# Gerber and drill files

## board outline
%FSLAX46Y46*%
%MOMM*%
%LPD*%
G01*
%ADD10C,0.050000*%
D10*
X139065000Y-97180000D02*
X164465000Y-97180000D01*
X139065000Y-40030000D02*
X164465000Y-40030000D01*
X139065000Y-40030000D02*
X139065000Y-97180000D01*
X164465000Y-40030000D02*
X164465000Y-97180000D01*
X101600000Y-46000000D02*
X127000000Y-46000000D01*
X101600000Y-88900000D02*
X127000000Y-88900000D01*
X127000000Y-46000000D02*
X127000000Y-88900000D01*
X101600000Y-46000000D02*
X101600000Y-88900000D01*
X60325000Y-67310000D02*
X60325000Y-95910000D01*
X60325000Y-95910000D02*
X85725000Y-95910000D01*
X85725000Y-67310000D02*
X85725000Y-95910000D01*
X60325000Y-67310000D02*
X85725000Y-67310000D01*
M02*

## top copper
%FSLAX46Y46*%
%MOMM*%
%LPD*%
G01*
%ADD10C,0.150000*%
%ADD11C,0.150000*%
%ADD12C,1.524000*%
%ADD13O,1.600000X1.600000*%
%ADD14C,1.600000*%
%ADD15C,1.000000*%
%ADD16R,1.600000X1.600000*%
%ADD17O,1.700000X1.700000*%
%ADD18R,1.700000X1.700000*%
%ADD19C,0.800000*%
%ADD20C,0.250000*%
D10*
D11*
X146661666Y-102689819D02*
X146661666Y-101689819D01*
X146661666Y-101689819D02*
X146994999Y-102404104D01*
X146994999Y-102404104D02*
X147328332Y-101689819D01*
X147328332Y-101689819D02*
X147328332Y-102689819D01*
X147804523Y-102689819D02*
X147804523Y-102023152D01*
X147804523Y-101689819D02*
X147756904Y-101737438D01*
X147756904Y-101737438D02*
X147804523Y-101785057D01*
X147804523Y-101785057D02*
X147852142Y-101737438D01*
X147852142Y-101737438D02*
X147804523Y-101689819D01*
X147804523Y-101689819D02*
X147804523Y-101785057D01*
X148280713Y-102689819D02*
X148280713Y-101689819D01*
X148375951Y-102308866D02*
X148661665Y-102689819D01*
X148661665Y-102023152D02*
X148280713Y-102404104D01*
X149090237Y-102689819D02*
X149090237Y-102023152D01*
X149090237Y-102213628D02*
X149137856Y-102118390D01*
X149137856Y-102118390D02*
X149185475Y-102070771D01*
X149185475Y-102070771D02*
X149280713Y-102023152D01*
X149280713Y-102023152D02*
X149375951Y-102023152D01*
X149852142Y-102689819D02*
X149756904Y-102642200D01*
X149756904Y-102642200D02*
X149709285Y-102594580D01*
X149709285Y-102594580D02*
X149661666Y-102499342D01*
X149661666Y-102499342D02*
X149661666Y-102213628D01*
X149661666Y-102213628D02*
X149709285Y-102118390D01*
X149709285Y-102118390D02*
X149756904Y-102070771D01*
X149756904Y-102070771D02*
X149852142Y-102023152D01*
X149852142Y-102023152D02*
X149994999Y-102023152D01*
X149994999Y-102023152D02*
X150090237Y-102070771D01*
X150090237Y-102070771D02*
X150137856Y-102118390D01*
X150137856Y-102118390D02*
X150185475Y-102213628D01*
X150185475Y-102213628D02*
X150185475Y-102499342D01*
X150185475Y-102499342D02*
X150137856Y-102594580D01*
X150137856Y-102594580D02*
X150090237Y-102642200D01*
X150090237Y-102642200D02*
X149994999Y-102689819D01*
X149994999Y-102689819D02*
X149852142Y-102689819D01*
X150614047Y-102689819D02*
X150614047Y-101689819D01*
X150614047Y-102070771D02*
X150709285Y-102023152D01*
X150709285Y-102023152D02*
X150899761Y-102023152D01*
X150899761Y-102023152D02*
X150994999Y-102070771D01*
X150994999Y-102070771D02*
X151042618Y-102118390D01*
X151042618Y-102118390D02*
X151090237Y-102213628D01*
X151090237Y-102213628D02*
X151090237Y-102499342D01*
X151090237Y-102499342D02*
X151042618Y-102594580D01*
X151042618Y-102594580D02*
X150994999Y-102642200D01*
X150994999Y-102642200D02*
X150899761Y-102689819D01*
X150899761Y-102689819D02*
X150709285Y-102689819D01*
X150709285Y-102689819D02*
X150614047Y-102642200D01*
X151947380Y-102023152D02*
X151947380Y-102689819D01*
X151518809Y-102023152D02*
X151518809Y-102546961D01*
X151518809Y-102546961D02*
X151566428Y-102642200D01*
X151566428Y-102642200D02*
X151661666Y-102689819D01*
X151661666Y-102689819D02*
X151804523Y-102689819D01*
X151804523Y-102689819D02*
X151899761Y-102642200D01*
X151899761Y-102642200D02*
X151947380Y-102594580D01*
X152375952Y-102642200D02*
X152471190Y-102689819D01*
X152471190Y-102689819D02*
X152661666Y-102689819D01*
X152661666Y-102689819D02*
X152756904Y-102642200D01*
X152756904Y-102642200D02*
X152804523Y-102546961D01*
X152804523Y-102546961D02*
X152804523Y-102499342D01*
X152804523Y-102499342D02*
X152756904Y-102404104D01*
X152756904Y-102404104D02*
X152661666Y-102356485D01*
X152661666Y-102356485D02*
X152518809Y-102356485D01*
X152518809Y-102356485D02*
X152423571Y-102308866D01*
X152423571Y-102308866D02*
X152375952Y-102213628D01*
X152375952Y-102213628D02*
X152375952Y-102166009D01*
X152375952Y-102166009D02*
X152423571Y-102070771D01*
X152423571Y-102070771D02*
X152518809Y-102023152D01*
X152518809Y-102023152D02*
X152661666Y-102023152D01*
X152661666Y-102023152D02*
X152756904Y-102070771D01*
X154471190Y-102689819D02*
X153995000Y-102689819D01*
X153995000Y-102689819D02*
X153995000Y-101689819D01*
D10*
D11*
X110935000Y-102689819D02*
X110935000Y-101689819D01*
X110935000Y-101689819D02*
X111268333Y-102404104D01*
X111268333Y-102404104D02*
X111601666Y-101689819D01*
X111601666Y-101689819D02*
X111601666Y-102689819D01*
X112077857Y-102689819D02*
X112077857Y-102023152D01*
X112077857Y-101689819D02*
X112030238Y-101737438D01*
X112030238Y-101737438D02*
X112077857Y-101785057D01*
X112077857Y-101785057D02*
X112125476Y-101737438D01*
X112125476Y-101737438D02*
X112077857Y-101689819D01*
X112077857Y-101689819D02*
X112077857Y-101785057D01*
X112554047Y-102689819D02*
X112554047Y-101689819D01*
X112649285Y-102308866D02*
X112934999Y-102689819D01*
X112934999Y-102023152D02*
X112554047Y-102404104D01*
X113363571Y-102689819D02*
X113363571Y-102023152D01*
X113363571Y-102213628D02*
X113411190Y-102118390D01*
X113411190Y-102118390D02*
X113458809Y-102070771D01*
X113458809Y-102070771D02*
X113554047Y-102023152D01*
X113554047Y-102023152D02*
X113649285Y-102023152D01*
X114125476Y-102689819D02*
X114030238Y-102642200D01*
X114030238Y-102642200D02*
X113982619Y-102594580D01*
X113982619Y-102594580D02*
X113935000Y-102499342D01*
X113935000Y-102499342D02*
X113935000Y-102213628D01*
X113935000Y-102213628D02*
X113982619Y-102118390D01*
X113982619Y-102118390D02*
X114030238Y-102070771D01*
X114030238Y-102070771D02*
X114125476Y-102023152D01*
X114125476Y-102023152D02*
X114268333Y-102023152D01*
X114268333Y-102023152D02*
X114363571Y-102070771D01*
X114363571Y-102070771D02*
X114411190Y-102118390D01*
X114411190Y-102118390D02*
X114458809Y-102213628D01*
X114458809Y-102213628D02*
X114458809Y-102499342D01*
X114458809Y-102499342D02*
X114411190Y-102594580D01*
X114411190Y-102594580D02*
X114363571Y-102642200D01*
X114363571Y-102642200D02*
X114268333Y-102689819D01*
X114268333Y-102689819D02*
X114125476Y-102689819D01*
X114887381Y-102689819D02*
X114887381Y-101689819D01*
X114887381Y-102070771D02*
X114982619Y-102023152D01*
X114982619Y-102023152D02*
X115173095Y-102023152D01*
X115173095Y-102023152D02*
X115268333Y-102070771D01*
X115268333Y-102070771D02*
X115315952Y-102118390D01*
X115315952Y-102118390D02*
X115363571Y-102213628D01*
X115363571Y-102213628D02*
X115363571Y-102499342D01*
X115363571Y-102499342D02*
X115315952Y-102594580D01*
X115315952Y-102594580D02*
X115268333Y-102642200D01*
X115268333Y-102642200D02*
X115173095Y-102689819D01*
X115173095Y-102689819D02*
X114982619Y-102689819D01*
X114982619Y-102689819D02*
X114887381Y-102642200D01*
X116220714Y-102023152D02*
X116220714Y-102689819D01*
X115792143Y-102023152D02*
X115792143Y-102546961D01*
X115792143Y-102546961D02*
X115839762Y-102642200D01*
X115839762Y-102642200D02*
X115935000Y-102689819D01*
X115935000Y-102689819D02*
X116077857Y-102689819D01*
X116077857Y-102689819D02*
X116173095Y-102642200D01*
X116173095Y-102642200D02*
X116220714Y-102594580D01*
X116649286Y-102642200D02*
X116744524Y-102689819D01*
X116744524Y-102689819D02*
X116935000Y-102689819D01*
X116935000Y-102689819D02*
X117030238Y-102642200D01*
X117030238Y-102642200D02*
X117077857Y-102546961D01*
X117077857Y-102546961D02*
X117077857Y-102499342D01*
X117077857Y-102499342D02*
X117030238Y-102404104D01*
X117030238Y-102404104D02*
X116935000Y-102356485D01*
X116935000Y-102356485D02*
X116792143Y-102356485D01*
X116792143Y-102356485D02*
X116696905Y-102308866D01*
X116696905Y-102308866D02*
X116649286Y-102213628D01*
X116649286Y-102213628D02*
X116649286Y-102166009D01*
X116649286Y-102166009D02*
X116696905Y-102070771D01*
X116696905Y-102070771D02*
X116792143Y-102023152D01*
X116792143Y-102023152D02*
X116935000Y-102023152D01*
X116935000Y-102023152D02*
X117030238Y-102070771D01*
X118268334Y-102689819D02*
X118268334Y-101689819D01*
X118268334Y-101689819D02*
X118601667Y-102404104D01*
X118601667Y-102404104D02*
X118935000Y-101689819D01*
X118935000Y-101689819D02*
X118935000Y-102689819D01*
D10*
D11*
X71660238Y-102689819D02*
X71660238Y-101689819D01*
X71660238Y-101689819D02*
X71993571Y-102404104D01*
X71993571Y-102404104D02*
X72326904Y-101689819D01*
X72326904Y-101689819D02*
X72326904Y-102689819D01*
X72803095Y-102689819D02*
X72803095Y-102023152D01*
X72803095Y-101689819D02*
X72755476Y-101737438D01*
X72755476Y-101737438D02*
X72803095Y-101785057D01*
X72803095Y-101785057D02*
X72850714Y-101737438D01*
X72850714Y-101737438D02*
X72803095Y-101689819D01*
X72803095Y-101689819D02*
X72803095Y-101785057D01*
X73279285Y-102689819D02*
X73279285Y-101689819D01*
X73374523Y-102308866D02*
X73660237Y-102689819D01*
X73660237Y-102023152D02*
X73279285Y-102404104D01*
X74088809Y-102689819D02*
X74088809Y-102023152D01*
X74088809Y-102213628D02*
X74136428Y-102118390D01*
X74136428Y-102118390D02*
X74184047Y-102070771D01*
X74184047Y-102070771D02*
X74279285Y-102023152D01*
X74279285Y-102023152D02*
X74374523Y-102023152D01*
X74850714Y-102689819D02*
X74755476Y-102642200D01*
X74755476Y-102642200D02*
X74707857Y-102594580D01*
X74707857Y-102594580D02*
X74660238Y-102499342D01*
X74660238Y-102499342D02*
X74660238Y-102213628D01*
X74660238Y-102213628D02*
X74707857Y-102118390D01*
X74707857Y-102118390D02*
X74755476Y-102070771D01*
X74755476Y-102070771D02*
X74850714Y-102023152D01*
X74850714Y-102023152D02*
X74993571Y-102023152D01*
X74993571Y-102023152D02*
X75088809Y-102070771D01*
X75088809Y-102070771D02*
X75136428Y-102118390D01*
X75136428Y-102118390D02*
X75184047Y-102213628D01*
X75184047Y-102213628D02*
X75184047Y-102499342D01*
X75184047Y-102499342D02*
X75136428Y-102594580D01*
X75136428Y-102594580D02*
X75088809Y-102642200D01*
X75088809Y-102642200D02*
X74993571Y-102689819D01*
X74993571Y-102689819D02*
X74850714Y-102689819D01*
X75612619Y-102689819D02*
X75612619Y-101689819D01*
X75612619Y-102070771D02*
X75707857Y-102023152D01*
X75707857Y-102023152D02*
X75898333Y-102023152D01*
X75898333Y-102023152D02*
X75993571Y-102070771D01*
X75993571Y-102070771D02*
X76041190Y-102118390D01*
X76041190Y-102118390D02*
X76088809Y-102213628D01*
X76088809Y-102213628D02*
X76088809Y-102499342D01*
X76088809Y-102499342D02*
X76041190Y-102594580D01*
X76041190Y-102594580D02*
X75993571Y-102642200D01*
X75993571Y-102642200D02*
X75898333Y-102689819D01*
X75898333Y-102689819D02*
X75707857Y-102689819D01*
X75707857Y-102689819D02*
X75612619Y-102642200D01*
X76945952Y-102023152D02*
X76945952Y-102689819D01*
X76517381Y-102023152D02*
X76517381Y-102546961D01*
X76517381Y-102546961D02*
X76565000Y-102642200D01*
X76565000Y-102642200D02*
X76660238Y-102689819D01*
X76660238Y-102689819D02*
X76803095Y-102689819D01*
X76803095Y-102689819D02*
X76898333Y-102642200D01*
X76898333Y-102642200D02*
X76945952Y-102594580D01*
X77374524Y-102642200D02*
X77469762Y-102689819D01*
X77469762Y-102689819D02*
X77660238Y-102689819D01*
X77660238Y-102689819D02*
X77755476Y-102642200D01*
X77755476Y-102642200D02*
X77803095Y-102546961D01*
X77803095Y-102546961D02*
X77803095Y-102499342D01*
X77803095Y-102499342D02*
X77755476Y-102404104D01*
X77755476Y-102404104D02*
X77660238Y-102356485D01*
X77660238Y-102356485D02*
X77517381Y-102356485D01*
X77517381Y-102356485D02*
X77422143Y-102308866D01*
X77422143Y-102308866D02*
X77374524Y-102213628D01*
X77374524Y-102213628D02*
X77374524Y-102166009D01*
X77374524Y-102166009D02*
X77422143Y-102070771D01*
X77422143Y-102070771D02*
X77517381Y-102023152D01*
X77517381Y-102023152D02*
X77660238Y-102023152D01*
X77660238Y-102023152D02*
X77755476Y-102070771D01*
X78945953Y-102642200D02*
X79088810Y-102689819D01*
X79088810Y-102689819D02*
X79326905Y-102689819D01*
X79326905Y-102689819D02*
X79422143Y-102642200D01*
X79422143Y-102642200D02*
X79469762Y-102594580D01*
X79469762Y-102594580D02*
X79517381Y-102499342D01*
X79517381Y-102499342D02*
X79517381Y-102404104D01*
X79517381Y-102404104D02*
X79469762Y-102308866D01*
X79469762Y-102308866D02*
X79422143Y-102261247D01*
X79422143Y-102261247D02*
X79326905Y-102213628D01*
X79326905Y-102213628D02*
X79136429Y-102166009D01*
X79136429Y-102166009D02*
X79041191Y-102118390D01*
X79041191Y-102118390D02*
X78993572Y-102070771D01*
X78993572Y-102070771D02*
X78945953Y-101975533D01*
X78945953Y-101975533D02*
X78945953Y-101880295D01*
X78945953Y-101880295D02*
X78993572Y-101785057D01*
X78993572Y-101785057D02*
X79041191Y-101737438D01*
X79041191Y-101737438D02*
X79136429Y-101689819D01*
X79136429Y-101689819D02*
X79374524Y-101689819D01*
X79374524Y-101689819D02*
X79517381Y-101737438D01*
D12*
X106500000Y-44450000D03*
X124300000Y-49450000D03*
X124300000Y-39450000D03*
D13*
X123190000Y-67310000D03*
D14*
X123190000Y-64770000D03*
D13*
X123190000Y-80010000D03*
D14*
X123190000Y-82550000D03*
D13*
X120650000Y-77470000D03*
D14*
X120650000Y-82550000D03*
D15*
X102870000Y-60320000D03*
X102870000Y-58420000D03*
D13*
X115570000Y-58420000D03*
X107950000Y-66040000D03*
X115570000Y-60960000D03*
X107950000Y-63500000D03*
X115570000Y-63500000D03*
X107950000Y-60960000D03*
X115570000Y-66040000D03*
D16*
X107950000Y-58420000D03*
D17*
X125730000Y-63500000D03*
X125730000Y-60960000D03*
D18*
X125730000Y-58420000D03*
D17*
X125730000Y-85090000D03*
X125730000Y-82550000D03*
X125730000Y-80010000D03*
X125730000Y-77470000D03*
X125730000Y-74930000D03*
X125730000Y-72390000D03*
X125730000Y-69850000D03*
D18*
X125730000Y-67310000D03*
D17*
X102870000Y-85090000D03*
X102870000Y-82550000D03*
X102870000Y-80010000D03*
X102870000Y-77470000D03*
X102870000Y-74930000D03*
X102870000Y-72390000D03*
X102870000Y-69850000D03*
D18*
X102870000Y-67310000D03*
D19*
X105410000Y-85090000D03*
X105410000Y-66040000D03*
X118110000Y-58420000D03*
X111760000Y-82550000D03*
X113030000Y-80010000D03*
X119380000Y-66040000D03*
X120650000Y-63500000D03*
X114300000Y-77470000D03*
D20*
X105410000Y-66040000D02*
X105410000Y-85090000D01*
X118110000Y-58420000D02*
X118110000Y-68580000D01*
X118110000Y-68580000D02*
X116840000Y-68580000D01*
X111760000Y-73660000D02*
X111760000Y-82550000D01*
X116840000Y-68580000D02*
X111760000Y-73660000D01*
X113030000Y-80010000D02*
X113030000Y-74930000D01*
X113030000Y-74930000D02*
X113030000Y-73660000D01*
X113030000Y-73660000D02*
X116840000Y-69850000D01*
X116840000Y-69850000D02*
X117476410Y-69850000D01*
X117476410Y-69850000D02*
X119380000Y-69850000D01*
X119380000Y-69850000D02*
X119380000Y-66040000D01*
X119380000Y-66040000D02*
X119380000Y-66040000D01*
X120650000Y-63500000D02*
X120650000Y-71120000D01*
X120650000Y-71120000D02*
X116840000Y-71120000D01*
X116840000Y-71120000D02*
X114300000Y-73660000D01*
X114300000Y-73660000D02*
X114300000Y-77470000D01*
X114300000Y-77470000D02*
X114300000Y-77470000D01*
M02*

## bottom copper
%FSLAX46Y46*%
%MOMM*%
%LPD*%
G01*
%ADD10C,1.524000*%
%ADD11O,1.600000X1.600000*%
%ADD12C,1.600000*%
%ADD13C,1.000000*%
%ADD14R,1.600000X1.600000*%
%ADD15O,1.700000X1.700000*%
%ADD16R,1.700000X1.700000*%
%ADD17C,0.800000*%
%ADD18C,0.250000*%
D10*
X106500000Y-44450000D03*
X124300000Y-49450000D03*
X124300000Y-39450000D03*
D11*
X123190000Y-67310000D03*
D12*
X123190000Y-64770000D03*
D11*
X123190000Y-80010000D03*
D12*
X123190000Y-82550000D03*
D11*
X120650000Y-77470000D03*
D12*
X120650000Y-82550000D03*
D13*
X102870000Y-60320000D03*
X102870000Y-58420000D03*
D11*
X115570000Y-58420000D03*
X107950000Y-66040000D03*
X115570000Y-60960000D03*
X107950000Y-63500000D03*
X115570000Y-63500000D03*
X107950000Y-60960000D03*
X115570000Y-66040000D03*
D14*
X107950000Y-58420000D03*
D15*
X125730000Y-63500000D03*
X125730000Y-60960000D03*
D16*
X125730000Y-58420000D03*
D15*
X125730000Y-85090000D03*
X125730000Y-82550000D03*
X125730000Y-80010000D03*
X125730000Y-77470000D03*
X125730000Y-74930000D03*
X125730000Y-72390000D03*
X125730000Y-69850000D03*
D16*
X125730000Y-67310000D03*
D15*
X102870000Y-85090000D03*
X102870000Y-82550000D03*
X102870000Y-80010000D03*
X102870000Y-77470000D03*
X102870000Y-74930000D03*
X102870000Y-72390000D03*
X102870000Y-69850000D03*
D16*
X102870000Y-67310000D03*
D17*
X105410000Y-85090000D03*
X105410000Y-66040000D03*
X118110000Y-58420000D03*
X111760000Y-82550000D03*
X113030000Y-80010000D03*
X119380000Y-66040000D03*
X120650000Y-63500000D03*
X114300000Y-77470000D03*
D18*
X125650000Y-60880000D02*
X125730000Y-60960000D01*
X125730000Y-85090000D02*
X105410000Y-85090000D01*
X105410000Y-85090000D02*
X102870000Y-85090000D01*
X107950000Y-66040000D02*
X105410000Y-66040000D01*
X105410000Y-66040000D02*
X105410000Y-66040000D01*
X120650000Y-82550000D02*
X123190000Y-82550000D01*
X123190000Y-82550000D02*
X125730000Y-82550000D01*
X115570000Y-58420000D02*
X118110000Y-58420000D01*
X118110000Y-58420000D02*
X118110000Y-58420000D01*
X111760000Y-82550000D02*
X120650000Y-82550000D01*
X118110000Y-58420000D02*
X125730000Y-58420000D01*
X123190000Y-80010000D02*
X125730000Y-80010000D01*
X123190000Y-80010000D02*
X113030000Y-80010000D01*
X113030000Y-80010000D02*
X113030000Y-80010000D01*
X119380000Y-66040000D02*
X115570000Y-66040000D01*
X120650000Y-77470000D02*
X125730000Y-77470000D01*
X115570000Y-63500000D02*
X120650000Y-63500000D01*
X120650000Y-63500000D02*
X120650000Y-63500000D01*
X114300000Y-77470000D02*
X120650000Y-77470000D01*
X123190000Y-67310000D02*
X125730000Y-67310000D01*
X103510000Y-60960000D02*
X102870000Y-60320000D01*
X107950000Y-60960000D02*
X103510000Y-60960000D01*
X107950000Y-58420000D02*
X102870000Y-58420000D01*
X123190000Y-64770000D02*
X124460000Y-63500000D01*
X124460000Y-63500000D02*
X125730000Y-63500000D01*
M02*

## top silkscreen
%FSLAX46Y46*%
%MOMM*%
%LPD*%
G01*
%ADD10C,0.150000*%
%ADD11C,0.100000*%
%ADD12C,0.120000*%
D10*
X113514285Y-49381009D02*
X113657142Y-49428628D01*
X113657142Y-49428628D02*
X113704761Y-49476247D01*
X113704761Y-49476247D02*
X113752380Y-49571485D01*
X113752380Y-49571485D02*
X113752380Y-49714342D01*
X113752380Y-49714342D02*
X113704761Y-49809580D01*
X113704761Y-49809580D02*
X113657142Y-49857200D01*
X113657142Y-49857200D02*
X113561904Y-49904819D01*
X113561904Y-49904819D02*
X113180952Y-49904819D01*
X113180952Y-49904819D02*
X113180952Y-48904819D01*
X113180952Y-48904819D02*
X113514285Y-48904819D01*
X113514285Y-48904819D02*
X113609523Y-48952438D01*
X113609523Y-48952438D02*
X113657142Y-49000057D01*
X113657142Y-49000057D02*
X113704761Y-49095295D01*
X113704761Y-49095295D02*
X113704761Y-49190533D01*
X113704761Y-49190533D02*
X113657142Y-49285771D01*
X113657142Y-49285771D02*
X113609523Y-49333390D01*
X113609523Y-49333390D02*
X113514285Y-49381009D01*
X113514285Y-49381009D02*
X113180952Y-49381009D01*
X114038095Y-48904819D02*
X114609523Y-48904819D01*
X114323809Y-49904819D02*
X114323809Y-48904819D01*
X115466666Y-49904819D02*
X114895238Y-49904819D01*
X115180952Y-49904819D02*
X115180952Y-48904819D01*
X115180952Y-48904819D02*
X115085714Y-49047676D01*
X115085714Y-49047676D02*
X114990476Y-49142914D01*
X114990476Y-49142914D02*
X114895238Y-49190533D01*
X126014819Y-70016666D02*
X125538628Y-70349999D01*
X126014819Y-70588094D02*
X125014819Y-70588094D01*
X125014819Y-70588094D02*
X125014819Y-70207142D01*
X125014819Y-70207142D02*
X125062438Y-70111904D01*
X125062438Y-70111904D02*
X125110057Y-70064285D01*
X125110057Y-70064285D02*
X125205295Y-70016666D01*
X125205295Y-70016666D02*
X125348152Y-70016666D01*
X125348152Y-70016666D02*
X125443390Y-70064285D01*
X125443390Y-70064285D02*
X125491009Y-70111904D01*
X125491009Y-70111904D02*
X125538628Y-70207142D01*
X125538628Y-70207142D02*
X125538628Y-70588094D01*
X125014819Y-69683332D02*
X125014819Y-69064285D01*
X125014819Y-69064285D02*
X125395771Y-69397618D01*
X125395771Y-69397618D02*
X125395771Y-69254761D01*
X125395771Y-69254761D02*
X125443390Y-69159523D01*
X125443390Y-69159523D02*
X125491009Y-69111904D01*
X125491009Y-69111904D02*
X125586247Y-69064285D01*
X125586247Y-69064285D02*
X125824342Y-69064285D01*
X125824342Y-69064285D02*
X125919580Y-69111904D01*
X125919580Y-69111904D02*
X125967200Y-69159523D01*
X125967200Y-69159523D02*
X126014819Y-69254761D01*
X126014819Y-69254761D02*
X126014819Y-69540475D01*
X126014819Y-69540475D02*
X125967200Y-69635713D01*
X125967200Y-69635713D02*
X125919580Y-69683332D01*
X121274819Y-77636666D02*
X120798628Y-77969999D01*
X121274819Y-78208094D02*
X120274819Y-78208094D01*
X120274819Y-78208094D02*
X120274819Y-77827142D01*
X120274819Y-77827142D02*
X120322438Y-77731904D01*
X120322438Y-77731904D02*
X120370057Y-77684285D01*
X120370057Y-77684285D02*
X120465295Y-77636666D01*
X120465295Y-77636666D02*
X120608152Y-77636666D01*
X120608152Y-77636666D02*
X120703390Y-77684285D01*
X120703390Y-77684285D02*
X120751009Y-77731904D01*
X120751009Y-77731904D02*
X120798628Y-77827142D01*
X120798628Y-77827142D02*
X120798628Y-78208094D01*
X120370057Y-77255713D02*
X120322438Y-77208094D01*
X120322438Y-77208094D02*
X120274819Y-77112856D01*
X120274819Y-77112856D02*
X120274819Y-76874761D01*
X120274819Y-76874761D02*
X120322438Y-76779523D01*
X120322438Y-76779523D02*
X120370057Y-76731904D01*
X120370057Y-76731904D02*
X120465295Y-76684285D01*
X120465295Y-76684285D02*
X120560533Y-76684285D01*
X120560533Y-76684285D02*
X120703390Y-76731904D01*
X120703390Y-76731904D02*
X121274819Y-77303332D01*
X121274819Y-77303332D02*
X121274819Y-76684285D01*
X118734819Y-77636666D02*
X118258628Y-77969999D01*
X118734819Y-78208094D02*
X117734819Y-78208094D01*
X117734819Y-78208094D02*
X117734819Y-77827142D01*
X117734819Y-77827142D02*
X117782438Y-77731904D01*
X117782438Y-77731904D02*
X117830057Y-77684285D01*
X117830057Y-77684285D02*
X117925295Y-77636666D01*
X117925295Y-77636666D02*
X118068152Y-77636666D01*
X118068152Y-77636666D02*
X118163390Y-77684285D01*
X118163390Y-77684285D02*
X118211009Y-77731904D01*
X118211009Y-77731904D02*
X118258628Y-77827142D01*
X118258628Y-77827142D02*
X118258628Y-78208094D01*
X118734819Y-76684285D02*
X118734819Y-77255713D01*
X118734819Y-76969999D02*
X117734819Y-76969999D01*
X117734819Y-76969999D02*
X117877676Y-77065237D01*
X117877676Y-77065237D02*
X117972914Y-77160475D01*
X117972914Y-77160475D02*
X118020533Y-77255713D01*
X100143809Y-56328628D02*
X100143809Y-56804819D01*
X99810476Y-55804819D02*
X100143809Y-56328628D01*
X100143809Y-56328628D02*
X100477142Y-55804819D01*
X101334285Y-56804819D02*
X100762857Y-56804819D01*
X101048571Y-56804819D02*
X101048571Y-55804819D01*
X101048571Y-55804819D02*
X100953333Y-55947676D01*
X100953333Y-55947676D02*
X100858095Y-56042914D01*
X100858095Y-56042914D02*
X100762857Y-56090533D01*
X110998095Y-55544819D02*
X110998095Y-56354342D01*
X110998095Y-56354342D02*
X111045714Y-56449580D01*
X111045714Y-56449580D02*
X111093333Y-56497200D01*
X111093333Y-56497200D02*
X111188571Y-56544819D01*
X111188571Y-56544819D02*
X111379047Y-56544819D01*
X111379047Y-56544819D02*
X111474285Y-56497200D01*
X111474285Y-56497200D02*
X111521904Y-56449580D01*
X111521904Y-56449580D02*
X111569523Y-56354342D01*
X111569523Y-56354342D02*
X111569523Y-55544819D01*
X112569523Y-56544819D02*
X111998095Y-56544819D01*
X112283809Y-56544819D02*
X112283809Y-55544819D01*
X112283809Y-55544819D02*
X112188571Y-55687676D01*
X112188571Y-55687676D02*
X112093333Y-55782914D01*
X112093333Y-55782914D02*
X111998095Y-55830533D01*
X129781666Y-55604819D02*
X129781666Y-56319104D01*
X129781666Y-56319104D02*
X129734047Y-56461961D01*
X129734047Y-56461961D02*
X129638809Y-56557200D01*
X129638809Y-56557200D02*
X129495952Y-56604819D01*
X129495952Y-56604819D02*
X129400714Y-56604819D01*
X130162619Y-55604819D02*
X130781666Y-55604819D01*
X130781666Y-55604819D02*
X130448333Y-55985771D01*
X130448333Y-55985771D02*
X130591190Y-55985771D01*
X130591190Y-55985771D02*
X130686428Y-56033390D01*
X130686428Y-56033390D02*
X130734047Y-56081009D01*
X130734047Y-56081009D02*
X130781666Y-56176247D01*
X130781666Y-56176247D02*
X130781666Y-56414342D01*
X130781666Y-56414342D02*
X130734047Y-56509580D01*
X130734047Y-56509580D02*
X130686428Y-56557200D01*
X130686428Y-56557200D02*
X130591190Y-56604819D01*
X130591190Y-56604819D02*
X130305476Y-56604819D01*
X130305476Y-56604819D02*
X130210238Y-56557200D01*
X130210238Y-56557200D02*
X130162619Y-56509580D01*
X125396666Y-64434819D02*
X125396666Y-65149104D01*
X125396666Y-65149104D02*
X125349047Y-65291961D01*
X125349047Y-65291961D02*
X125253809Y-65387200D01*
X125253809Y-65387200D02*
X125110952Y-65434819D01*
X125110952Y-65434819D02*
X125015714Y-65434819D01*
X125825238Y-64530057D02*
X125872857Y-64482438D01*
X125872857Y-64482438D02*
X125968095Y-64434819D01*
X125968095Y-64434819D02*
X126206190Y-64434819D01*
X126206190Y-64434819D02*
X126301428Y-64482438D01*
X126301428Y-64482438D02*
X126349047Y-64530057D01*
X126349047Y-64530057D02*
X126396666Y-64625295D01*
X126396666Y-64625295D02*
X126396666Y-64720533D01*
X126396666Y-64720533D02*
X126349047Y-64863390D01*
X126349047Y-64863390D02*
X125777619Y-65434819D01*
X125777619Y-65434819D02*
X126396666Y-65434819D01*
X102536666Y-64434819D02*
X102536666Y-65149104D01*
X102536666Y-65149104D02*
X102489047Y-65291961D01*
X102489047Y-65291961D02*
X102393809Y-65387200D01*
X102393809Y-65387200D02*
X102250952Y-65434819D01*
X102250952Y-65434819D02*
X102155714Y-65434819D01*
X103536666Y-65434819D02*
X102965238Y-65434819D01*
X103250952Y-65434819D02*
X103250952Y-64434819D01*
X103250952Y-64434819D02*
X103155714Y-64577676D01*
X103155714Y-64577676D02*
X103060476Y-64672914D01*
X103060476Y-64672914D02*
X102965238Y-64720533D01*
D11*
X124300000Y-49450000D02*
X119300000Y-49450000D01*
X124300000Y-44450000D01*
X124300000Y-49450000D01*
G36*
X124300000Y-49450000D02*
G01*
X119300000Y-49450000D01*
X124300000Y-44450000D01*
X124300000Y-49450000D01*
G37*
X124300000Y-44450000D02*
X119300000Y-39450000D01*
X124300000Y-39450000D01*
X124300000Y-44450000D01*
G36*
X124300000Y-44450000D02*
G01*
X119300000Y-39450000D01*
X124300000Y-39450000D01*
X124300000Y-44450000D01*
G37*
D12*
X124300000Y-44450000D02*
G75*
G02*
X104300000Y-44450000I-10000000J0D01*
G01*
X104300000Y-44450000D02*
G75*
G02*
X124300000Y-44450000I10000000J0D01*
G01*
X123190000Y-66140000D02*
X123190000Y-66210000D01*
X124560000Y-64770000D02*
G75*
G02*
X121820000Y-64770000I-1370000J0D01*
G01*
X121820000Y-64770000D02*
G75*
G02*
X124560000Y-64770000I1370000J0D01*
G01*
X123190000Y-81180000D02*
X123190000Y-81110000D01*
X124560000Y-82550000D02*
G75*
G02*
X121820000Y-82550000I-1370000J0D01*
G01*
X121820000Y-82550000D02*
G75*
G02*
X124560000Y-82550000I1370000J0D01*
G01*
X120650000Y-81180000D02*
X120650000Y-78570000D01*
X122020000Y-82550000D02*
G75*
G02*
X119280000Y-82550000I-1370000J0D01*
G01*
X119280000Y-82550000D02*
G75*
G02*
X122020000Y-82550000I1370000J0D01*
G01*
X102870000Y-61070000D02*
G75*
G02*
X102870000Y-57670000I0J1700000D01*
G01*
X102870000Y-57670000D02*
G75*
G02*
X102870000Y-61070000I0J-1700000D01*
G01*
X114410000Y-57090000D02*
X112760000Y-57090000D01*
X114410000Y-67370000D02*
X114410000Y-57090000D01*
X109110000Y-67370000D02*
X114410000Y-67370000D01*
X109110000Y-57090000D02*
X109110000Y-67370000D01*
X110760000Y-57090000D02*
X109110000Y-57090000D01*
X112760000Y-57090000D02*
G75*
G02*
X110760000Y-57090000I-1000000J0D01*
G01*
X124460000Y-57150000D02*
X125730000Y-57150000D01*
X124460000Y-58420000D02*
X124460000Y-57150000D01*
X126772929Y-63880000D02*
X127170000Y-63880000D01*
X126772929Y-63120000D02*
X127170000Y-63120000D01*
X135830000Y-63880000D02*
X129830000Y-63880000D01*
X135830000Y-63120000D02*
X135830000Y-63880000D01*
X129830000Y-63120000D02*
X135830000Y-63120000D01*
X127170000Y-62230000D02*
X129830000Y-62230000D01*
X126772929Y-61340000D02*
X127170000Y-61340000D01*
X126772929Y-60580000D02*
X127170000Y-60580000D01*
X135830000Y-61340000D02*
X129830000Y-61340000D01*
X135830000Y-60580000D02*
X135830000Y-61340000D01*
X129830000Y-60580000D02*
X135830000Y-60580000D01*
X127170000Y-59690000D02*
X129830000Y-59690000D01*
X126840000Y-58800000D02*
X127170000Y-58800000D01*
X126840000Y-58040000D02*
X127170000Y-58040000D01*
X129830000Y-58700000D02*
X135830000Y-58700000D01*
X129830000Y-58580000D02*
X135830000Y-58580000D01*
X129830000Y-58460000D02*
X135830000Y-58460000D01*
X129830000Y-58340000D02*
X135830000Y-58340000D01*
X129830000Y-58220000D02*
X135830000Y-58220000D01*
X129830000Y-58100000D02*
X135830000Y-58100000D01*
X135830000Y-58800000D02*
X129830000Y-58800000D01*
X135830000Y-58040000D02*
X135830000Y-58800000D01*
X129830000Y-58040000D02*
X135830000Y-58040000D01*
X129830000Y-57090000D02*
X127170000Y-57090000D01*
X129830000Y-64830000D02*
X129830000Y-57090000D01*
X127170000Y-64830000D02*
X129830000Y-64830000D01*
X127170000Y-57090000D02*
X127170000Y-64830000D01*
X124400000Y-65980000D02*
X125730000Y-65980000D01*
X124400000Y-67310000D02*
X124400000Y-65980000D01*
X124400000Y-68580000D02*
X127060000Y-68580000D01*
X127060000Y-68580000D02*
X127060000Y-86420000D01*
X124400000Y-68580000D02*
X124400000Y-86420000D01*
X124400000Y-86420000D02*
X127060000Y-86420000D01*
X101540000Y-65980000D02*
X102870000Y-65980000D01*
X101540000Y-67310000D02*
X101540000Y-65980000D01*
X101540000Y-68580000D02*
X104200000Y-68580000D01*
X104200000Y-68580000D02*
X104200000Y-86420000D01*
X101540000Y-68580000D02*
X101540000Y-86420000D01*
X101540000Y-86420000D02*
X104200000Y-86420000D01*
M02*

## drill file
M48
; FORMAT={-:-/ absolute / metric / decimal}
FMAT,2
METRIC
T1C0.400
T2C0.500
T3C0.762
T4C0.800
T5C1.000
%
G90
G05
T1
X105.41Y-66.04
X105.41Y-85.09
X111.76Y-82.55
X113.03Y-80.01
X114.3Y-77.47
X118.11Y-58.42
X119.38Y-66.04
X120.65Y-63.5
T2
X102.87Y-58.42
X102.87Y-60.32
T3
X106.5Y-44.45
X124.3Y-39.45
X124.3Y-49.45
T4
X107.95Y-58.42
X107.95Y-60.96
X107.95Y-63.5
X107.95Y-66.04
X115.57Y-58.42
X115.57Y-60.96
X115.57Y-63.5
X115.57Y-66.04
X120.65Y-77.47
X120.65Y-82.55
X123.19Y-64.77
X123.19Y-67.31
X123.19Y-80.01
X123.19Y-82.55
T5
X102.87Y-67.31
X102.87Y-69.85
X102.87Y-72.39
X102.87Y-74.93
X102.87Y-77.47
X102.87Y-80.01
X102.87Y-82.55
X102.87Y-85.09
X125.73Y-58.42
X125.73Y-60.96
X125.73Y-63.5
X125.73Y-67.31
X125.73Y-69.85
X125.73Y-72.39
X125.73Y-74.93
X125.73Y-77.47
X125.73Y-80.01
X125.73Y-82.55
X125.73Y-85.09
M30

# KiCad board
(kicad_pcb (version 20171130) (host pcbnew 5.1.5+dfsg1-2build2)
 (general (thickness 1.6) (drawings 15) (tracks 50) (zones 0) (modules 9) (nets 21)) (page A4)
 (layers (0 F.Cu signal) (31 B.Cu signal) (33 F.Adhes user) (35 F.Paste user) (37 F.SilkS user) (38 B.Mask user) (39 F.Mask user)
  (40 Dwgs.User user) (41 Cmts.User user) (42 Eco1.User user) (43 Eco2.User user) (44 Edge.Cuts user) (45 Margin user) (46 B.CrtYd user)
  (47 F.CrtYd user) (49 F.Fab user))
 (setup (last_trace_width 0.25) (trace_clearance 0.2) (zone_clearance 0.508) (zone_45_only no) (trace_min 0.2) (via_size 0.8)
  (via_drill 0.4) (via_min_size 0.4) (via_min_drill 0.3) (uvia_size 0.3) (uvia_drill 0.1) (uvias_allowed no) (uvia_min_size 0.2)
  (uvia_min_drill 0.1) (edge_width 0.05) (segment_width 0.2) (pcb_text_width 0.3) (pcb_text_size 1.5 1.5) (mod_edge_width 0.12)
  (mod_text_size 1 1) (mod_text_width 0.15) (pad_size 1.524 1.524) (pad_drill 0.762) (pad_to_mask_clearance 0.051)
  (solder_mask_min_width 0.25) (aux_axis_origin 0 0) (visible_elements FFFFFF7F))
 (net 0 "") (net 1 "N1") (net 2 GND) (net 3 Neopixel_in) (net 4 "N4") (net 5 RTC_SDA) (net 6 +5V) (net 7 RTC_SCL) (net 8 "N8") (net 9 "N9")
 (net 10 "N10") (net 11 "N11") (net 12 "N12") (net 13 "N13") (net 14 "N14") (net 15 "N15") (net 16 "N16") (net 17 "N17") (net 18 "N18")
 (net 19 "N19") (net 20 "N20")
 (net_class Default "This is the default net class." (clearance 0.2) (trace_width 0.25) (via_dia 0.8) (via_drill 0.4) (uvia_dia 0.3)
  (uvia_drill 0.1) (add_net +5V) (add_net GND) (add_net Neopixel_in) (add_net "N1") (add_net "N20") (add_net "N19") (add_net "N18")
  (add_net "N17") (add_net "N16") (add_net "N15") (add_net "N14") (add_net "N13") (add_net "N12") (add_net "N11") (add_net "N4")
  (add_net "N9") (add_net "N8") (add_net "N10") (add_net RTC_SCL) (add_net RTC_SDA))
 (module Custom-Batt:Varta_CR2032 (layer F.Cu) (at 114.3 44.45)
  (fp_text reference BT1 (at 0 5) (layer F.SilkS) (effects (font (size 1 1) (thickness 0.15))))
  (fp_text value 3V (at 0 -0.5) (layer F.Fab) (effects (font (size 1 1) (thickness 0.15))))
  (fp_poly (pts (xy 10 5) (xy 5 5) (xy 10 0)) (layer F.SilkS) (width 0.1))
  (fp_poly (pts (xy 10 0) (xy 5 -5) (xy 10 -5)) (layer F.SilkS) (width 0.1))
  (fp_circle (center 0 0) (end 10 0) (layer F.SilkS) (width 0.12))
  (pad 1 thru_hole circle (at -7.8 0) (size 1.524 1.524) (drill 0.762) (layers *.Cu *.Mask) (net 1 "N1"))
  (pad 2 thru_hole circle (at 10 5) (size 1.524 1.524) (drill 0.762) (layers *.Cu *.Mask) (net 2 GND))
  (pad 2 thru_hole circle (at 10 -5) (size 1.524 1.524) (drill 0.762) (layers *.Cu *.Mask) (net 2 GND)))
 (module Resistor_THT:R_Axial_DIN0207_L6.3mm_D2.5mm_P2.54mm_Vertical (layer F.Cu) (at 123.19 64.77 270)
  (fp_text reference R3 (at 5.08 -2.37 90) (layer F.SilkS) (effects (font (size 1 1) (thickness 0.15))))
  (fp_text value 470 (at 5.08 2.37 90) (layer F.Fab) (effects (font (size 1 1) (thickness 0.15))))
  (fp_line (start 1.37 0) (end 1.44 0) (layer F.SilkS) (width 0.12))
  (fp_circle (center 0 0) (end 1.37 0) (layer F.SilkS) (width 0.12))
  (pad 2 thru_hole oval (at 2.54 0 270) (size 1.6 1.6) (drill 0.8) (layers *.Cu *.Mask) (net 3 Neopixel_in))
  (pad 1 thru_hole circle (at 0 0 270) (size 1.6 1.6) (drill 0.8) (layers *.Cu *.Mask) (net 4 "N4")))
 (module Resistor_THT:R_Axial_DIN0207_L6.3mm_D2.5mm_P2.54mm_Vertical (layer F.Cu) (at 123.19 82.55 90)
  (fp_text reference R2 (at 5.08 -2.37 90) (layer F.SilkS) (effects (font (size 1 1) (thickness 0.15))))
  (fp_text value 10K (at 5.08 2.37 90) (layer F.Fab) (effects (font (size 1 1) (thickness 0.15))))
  (fp_line (start 1.37 0) (end 1.44 0) (layer F.SilkS) (width 0.12))
  (fp_circle (center 0 0) (end 1.37 0) (layer F.SilkS) (width 0.12))
  (pad 2 thru_hole oval (at 2.54 0 90) (size 1.6 1.6) (drill 0.8) (layers *.Cu *.Mask) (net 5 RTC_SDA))
  (pad 1 thru_hole circle (at 0 0 90) (size 1.6 1.6) (drill 0.8) (layers *.Cu *.Mask) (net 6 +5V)))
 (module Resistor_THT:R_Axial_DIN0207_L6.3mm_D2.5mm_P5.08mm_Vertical (layer F.Cu) (at 120.65 82.55 90)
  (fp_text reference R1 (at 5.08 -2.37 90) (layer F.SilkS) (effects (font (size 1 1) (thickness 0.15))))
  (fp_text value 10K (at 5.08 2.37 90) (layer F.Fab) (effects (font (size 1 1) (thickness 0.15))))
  (fp_line (start 1.37 0) (end 3.98 0) (layer F.SilkS) (width 0.12))
  (fp_circle (center 0 0) (end 1.37 0) (layer F.SilkS) (width 0.12))
  (pad 2 thru_hole oval (at 5.08 0 90) (size 1.6 1.6) (drill 0.8) (layers *.Cu *.Mask) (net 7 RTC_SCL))
  (pad 1 thru_hole circle (at 0 0 90) (size 1.6 1.6) (drill 0.8) (layers *.Cu *.Mask) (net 6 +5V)))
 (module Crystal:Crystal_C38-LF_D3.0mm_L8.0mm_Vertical (layer F.Cu) (at 102.87 58.42 270)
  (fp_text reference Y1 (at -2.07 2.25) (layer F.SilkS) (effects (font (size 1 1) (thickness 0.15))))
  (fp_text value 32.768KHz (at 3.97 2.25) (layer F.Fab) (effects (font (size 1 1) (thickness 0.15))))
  (fp_arc (start 0.95 0) (end -0.75 0) (angle -180) (layer F.SilkS) (width 0.12))
  (fp_arc (start 0.95 0) (end -0.75 0) (angle 180) (layer F.SilkS) (width 0.12))
  (pad 2 thru_hole circle (at 1.9 0 270) (size 1 1) (drill 0.5) (layers *.Cu *.Mask) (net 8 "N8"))
  (pad 1 thru_hole circle (at 0 0 270) (size 1 1) (drill 0.5) (layers *.Cu *.Mask) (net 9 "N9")))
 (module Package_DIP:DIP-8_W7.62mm (layer F.Cu) (at 107.95 58.42)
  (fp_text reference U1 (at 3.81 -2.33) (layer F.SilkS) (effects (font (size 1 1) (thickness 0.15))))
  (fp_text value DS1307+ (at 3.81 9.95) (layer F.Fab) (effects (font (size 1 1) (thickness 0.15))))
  (fp_line (start 6.46 -1.33) (end 4.81 -1.33) (layer F.SilkS) (width 0.12))
  (fp_line (start 6.46 8.95) (end 6.46 -1.33) (layer F.SilkS) (width 0.12))
  (fp_line (start 1.16 8.95) (end 6.46 8.95) (layer F.SilkS) (width 0.12))
  (fp_line (start 1.16 -1.33) (end 1.16 8.95) (layer F.SilkS) (width 0.12))
  (fp_line (start 2.81 -1.33) (end 1.16 -1.33) (layer F.SilkS) (width 0.12))
  (fp_arc (start 3.81 -1.33) (end 2.81 -1.33) (angle -180) (layer F.SilkS) (width 0.12))
  (pad 8 thru_hole oval (at 7.62 0) (size 1.6 1.6) (drill 0.8) (layers *.Cu *.Mask) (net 6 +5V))
  (pad 4 thru_hole oval (at 0 7.62) (size 1.6 1.6) (drill 0.8) (layers *.Cu *.Mask) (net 2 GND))
  (pad 7 thru_hole oval (at 7.62 2.54) (size 1.6 1.6) (drill 0.8) (layers *.Cu *.Mask) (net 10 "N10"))
  (pad 3 thru_hole oval (at 0 5.08) (size 1.6 1.6) (drill 0.8) (layers *.Cu *.Mask) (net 1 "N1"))
  (pad 6 thru_hole oval (at 7.62 5.08) (size 1.6 1.6) (drill 0.8) (layers *.Cu *.Mask) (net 7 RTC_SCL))
  (pad 2 thru_hole oval (at 0 2.54) (size 1.6 1.6) (drill 0.8) (layers *.Cu *.Mask) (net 8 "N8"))
  (pad 5 thru_hole oval (at 7.62 7.62) (size 1.6 1.6) (drill 0.8) (layers *.Cu *.Mask) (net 5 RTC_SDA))
  (pad 1 thru_hole rect (at 0 0) (size 1.6 1.6) (drill 0.8) (layers *.Cu *.Mask) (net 9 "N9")))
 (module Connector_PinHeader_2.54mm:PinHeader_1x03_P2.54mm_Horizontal (layer F.Cu) (at 125.73 58.42)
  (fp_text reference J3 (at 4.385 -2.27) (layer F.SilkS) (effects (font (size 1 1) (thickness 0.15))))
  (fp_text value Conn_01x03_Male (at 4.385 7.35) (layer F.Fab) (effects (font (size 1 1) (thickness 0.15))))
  (fp_line (start -1.27 -1.27) (end 0 -1.27) (layer F.SilkS) (width 0.12))
  (fp_line (start -1.27 0) (end -1.27 -1.27) (layer F.SilkS) (width 0.12))
  (fp_line (start 1.042929 5.46) (end 1.44 5.46) (layer F.SilkS) (width 0.12))
  (fp_line (start 1.042929 4.7) (end 1.44 4.7) (layer F.SilkS) (width 0.12))
  (fp_line (start 10.1 5.46) (end 4.1 5.46) (layer F.SilkS) (width 0.12))
  (fp_line (start 10.1 4.7) (end 10.1 5.46) (layer F.SilkS) (width 0.12))
  (fp_line (start 4.1 4.7) (end 10.1 4.7) (layer F.SilkS) (width 0.12))
  (fp_line (start 1.44 3.81) (end 4.1 3.81) (layer F.SilkS) (width 0.12))
  (fp_line (start 1.042929 2.92) (end 1.44 2.92) (layer F.SilkS) (width 0.12))
  (fp_line (start 1.042929 2.16) (end 1.44 2.16) (layer F.SilkS) (width 0.12))
  (fp_line (start 10.1 2.92) (end 4.1 2.92) (layer F.SilkS) (width 0.12))
  (fp_line (start 10.1 2.16) (end 10.1 2.92) (layer F.SilkS) (width 0.12))
  (fp_line (start 4.1 2.16) (end 10.1 2.16) (layer F.SilkS) (width 0.12))
  (fp_line (start 1.44 1.27) (end 4.1 1.27) (layer F.SilkS) (width 0.12))
  (fp_line (start 1.11 0.38) (end 1.44 0.38) (layer F.SilkS) (width 0.12))
  (fp_line (start 1.11 -0.38) (end 1.44 -0.38) (layer F.SilkS) (width 0.12))
  (fp_line (start 4.1 0.28) (end 10.1 0.28) (layer F.SilkS) (width 0.12))
  (fp_line (start 4.1 0.16) (end 10.1 0.16) (layer F.SilkS) (width 0.12))
  (fp_line (start 4.1 0.04) (end 10.1 0.04) (layer F.SilkS) (width 0.12))
  (fp_line (start 4.1 -0.08) (end 10.1 -0.08) (layer F.SilkS) (width 0.12))
  (fp_line (start 4.1 -0.2) (end 10.1 -0.2) (layer F.SilkS) (width 0.12))
  (fp_line (start 4.1 -0.32) (end 10.1 -0.32) (layer F.SilkS) (width 0.12))
  (fp_line (start 10.1 0.38) (end 4.1 0.38) (layer F.SilkS) (width 0.12))
  (fp_line (start 10.1 -0.38) (end 10.1 0.38) (layer F.SilkS) (width 0.12))
  (fp_line (start 4.1 -0.38) (end 10.1 -0.38) (layer F.SilkS) (width 0.12))
  (fp_line (start 4.1 -1.33) (end 1.44 -1.33) (layer F.SilkS) (width 0.12))
  (fp_line (start 4.1 6.41) (end 4.1 -1.33) (layer F.SilkS) (width 0.12))
  (fp_line (start 1.44 6.41) (end 4.1 6.41) (layer F.SilkS) (width 0.12))
  (fp_line (start 1.44 -1.33) (end 1.44 6.41) (layer F.SilkS) (width 0.12))
  (pad 3 thru_hole oval (at 0 5.08) (size 1.7 1.7) (drill 1) (layers *.Cu *.Mask) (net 4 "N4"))
  (pad 2 thru_hole oval (at 0 2.54) (size 1.7 1.7) (drill 1) (layers *.Cu *.Mask) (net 2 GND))
  (pad 1 thru_hole rect (at 0 0) (size 1.7 1.7) (drill 1) (layers *.Cu *.Mask) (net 6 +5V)))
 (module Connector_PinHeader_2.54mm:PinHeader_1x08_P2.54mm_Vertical (layer F.Cu) (at 125.73 67.31)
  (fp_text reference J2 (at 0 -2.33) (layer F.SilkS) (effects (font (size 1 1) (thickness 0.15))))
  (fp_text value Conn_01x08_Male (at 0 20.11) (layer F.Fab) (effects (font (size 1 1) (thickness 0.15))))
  (fp_line (start -1.33 -1.33) (end 0 -1.33) (layer F.SilkS) (width 0.12))
  (fp_line (start -1.33 0) (end -1.33 -1.33) (layer F.SilkS) (width 0.12))
  (fp_line (start -1.33 1.27) (end 1.33 1.27) (layer F.SilkS) (width 0.12))
  (fp_line (start 1.33 1.27) (end 1.33 19.11) (layer F.SilkS) (width 0.12))
  (fp_line (start -1.33 1.27) (end -1.33 19.11) (layer F.SilkS) (width 0.12))
  (fp_line (start -1.33 19.11) (end 1.33 19.11) (layer F.SilkS) (width 0.12))
  (pad 8 thru_hole oval (at 0 17.78) (size 1.7 1.7) (drill 1) (layers *.Cu *.Mask) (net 2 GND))
  (pad 7 thru_hole oval (at 0 15.24) (size 1.7 1.7) (drill 1) (layers *.Cu *.Mask) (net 6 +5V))
  (pad 6 thru_hole oval (at 0 12.7) (size 1.7 1.7) (drill 1) (layers *.Cu *.Mask) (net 5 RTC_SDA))
  (pad 5 thru_hole oval (at 0 10.16) (size 1.7 1.7) (drill 1) (layers *.Cu *.Mask) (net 7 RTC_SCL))
  (pad 4 thru_hole oval (at 0 7.62) (size 1.7 1.7) (drill 1) (layers *.Cu *.Mask) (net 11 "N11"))
  (pad 3 thru_hole oval (at 0 5.08) (size 1.7 1.7) (drill 1) (layers *.Cu *.Mask) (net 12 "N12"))
  (pad 2 thru_hole oval (at 0 2.54) (size 1.7 1.7) (drill 1) (layers *.Cu *.Mask) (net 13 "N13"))
  (pad 1 thru_hole rect (at 0 0) (size 1.7 1.7) (drill 1) (layers *.Cu *.Mask) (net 3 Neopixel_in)))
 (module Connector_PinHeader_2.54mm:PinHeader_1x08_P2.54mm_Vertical (layer F.Cu) (at 102.87 67.31)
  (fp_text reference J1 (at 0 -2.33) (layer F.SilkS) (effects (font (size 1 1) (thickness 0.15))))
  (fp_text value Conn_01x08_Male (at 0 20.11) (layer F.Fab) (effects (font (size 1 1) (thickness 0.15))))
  (fp_line (start -1.33 -1.33) (end 0 -1.33) (layer F.SilkS) (width 0.12))
  (fp_line (start -1.33 0) (end -1.33 -1.33) (layer F.SilkS) (width 0.12))
  (fp_line (start -1.33 1.27) (end 1.33 1.27) (layer F.SilkS) (width 0.12))
  (fp_line (start 1.33 1.27) (end 1.33 19.11) (layer F.SilkS) (width 0.12))
  (fp_line (start -1.33 1.27) (end -1.33 19.11) (layer F.SilkS) (width 0.12))
  (fp_line (start -1.33 19.11) (end 1.33 19.11) (layer F.SilkS) (width 0.12))
  (pad 8 thru_hole oval (at 0 17.78) (size 1.7 1.7) (drill 1) (layers *.Cu *.Mask) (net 2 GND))
  (pad 7 thru_hole oval (at 0 15.24) (size 1.7 1.7) (drill 1) (layers *.Cu *.Mask) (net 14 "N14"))
  (pad 6 thru_hole oval (at 0 12.7) (size 1.7 1.7) (drill 1) (layers *.Cu *.Mask) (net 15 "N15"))
  (pad 5 thru_hole oval (at 0 10.16) (size 1.7 1.7) (drill 1) (layers *.Cu *.Mask) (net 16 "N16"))
  (pad 4 thru_hole oval (at 0 7.62) (size 1.7 1.7) (drill 1) (layers *.Cu *.Mask) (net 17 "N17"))
  (pad 3 thru_hole oval (at 0 5.08) (size 1.7 1.7) (drill 1) (layers *.Cu *.Mask) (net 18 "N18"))
  (pad 2 thru_hole oval (at 0 2.54) (size 1.7 1.7) (drill 1) (layers *.Cu *.Mask) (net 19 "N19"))
  (pad 1 thru_hole rect (at 0 0) (size 1.7 1.7) (drill 1) (layers *.Cu *.Mask) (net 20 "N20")))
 (gr_line (start 139.065 97.18) (end 164.465 97.18) (layer Edge.Cuts) (width 0.05))
 (gr_line (start 139.065 40.03) (end 164.465 40.03) (layer Edge.Cuts) (width 0.05))
 (gr_line (start 139.065 40.03) (end 139.065 97.18) (layer Edge.Cuts) (width 0.05))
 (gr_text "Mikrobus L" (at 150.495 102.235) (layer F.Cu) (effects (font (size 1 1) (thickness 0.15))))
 (gr_line (start 164.465 40.03) (end 164.465 97.18) (layer Edge.Cuts) (width 0.05))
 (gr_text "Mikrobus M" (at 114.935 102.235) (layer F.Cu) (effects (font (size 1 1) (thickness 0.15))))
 (gr_line (start 101.6 46) (end 127 46) (layer Edge.Cuts) (width 0.05))
 (gr_line (start 101.6 88.9) (end 127 88.9) (layer Edge.Cuts) (width 0.05))
 (gr_line (start 127 46) (end 127 88.9) (layer Edge.Cuts) (width 0.05))
 (gr_line (start 101.6 46) (end 101.6 88.9) (layer Edge.Cuts) (width 0.05))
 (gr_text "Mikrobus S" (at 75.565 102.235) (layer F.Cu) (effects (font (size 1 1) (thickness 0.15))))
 (gr_line (start 60.325 67.31) (end 60.325 95.91) (layer Edge.Cuts) (width 0.05))
 (gr_line (start 60.325 95.91) (end 85.725 95.91) (layer Edge.Cuts) (width 0.05))
 (gr_line (start 85.725 67.31) (end 85.725 95.91) (layer Edge.Cuts) (width 0.05))
 (gr_line (start 60.325 67.31) (end 85.725 67.31) (layer Edge.Cuts) (width 0.05))
 (segment (start 125.65 60.88) (end 125.73 60.96) (width 0.25) (layer B.Cu) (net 2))
 (segment (start 125.73 85.09) (end 105.41 85.09) (width 0.25) (layer B.Cu) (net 2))
 (segment (start 105.41 85.09) (end 102.87 85.09) (width 0.25) (layer B.Cu) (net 2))
 (via (at 105.41 85.09) (size 0.8) (drill 0.4) (layers F.Cu B.Cu) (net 2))
 (segment (start 107.95 66.04) (end 105.41 66.04) (width 0.25) (layer B.Cu) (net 2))
 (segment (start 105.41 66.04) (end 105.41 66.04) (width 0.25) (layer B.Cu) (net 2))
 (via (at 105.41 66.04) (size 0.8) (drill 0.4) (layers F.Cu B.Cu) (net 2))
 (segment (start 105.41 66.04) (end 105.41 85.09) (width 0.25) (layer F.Cu) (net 2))
 (segment (start 120.65 82.55) (end 123.19 82.55) (width 0.25) (layer B.Cu) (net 6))
 (segment (start 123.19 82.55) (end 125.73 82.55) (width 0.25) (layer B.Cu) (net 6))
 (segment (start 115.57 58.42) (end 118.11 58.42) (width 0.25) (layer B.Cu) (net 6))
 (segment (start 118.11 58.42) (end 118.11 58.42) (width 0.25) (layer B.Cu) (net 6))
 (via (at 118.11 58.42) (size 0.8) (drill 0.4) (layers F.Cu B.Cu) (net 6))
 (via (at 111.76 82.55) (size 0.8) (drill 0.4) (layers F.Cu B.Cu) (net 6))
 (segment (start 118.11 58.42) (end 118.11 68.58) (width 0.25) (layer F.Cu) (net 6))
 (segment (start 118.11 68.58) (end 116.84 68.58) (width 0.25) (layer F.Cu) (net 6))
 (segment (start 111.76 73.66) (end 111.76 82.55) (width 0.25) (layer F.Cu) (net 6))
 (segment (start 116.84 68.58) (end 111.76 73.66) (width 0.25) (layer F.Cu) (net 6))
 (segment (start 111.76 82.55) (end 120.65 82.55) (width 0.25) (layer B.Cu) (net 6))
 (segment (start 118.11 58.42) (end 125.73 58.42) (width 0.25) (layer B.Cu) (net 6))
 (segment (start 123.19 80.01) (end 125.73 80.01) (width 0.25) (layer B.Cu) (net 5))
 (segment (start 123.19 80.01) (end 113.03 80.01) (width 0.25) (layer B.Cu) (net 5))
 (segment (start 113.03 80.01) (end 113.03 80.01) (width 0.25) (layer B.Cu) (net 5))
 (via (at 113.03 80.01) (size 0.8) (drill 0.4) (layers F.Cu B.Cu) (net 5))
 (segment (start 113.03 80.01) (end 113.03 74.93) (width 0.25) (layer F.Cu) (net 5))
 (segment (start 113.03 74.93) (end 113.03 73.66) (width 0.25) (layer F.Cu) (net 5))
 (segment (start 113.03 73.66) (end 116.84 69.85) (width 0.25) (layer F.Cu) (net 5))
 (segment (start 116.84 69.85) (end 117.47641 69.85) (width 0.25) (layer F.Cu) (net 5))
 (segment (start 117.47641 69.85) (end 119.38 69.85) (width 0.25) (layer F.Cu) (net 5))
 (segment (start 119.38 69.85) (end 119.38 66.04) (width 0.25) (layer F.Cu) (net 5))
 (segment (start 119.38 66.04) (end 119.38 66.04) (width 0.25) (layer F.Cu) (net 5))
 (via (at 119.38 66.04) (size 0.8) (drill 0.4) (layers F.Cu B.Cu) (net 5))
 (segment (start 119.38 66.04) (end 115.57 66.04) (width 0.25) (layer B.Cu) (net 5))
 (segment (start 120.65 77.47) (end 125.73 77.47) (width 0.25) (layer B.Cu) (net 7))
 (segment (start 115.57 63.5) (end 120.65 63.5) (width 0.25) (layer B.Cu) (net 7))
 (segment (start 120.65 63.5) (end 120.65 63.5) (width 0.25) (layer B.Cu) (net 7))
 (via (at 120.65 63.5) (size 0.8) (drill 0.4) (layers F.Cu B.Cu) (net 7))
 (segment (start 120.65 63.5) (end 120.65 71.12) (width 0.25) (layer F.Cu) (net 7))
 (segment (start 120.65 71.12) (end 116.84 71.12) (width 0.25) (layer F.Cu) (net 7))
 (segment (start 116.84 71.12) (end 114.3 73.66) (width 0.25) (layer F.Cu) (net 7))
 (segment (start 114.3 73.66) (end 114.3 77.47) (width 0.25) (layer F.Cu) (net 7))
 (segment (start 114.3 77.47) (end 114.3 77.47) (width 0.25) (layer F.Cu) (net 7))
 (via (at 114.3 77.47) (size 0.8) (drill 0.4) (layers F.Cu B.Cu) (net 7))
 (segment (start 114.3 77.47) (end 120.65 77.47) (width 0.25) (layer B.Cu) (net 7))
 (segment (start 123.19 67.31) (end 125.73 67.31) (width 0.25) (layer B.Cu) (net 3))
 (segment (start 103.51 60.96) (end 102.87 60.32) (width 0.25) (layer B.Cu) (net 8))
 (segment (start 107.95 60.96) (end 103.51 60.96) (width 0.25) (layer B.Cu) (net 8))
 (segment (start 107.95 58.42) (end 102.87 58.42) (width 0.25) (layer B.Cu) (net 9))
 (segment (start 123.19 64.77) (end 124.46 63.5) (width 0.25) (layer B.Cu) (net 4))
 (segment (start 124.46 63.5) (end 125.73 63.5) (width 0.25) (layer B.Cu) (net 4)))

